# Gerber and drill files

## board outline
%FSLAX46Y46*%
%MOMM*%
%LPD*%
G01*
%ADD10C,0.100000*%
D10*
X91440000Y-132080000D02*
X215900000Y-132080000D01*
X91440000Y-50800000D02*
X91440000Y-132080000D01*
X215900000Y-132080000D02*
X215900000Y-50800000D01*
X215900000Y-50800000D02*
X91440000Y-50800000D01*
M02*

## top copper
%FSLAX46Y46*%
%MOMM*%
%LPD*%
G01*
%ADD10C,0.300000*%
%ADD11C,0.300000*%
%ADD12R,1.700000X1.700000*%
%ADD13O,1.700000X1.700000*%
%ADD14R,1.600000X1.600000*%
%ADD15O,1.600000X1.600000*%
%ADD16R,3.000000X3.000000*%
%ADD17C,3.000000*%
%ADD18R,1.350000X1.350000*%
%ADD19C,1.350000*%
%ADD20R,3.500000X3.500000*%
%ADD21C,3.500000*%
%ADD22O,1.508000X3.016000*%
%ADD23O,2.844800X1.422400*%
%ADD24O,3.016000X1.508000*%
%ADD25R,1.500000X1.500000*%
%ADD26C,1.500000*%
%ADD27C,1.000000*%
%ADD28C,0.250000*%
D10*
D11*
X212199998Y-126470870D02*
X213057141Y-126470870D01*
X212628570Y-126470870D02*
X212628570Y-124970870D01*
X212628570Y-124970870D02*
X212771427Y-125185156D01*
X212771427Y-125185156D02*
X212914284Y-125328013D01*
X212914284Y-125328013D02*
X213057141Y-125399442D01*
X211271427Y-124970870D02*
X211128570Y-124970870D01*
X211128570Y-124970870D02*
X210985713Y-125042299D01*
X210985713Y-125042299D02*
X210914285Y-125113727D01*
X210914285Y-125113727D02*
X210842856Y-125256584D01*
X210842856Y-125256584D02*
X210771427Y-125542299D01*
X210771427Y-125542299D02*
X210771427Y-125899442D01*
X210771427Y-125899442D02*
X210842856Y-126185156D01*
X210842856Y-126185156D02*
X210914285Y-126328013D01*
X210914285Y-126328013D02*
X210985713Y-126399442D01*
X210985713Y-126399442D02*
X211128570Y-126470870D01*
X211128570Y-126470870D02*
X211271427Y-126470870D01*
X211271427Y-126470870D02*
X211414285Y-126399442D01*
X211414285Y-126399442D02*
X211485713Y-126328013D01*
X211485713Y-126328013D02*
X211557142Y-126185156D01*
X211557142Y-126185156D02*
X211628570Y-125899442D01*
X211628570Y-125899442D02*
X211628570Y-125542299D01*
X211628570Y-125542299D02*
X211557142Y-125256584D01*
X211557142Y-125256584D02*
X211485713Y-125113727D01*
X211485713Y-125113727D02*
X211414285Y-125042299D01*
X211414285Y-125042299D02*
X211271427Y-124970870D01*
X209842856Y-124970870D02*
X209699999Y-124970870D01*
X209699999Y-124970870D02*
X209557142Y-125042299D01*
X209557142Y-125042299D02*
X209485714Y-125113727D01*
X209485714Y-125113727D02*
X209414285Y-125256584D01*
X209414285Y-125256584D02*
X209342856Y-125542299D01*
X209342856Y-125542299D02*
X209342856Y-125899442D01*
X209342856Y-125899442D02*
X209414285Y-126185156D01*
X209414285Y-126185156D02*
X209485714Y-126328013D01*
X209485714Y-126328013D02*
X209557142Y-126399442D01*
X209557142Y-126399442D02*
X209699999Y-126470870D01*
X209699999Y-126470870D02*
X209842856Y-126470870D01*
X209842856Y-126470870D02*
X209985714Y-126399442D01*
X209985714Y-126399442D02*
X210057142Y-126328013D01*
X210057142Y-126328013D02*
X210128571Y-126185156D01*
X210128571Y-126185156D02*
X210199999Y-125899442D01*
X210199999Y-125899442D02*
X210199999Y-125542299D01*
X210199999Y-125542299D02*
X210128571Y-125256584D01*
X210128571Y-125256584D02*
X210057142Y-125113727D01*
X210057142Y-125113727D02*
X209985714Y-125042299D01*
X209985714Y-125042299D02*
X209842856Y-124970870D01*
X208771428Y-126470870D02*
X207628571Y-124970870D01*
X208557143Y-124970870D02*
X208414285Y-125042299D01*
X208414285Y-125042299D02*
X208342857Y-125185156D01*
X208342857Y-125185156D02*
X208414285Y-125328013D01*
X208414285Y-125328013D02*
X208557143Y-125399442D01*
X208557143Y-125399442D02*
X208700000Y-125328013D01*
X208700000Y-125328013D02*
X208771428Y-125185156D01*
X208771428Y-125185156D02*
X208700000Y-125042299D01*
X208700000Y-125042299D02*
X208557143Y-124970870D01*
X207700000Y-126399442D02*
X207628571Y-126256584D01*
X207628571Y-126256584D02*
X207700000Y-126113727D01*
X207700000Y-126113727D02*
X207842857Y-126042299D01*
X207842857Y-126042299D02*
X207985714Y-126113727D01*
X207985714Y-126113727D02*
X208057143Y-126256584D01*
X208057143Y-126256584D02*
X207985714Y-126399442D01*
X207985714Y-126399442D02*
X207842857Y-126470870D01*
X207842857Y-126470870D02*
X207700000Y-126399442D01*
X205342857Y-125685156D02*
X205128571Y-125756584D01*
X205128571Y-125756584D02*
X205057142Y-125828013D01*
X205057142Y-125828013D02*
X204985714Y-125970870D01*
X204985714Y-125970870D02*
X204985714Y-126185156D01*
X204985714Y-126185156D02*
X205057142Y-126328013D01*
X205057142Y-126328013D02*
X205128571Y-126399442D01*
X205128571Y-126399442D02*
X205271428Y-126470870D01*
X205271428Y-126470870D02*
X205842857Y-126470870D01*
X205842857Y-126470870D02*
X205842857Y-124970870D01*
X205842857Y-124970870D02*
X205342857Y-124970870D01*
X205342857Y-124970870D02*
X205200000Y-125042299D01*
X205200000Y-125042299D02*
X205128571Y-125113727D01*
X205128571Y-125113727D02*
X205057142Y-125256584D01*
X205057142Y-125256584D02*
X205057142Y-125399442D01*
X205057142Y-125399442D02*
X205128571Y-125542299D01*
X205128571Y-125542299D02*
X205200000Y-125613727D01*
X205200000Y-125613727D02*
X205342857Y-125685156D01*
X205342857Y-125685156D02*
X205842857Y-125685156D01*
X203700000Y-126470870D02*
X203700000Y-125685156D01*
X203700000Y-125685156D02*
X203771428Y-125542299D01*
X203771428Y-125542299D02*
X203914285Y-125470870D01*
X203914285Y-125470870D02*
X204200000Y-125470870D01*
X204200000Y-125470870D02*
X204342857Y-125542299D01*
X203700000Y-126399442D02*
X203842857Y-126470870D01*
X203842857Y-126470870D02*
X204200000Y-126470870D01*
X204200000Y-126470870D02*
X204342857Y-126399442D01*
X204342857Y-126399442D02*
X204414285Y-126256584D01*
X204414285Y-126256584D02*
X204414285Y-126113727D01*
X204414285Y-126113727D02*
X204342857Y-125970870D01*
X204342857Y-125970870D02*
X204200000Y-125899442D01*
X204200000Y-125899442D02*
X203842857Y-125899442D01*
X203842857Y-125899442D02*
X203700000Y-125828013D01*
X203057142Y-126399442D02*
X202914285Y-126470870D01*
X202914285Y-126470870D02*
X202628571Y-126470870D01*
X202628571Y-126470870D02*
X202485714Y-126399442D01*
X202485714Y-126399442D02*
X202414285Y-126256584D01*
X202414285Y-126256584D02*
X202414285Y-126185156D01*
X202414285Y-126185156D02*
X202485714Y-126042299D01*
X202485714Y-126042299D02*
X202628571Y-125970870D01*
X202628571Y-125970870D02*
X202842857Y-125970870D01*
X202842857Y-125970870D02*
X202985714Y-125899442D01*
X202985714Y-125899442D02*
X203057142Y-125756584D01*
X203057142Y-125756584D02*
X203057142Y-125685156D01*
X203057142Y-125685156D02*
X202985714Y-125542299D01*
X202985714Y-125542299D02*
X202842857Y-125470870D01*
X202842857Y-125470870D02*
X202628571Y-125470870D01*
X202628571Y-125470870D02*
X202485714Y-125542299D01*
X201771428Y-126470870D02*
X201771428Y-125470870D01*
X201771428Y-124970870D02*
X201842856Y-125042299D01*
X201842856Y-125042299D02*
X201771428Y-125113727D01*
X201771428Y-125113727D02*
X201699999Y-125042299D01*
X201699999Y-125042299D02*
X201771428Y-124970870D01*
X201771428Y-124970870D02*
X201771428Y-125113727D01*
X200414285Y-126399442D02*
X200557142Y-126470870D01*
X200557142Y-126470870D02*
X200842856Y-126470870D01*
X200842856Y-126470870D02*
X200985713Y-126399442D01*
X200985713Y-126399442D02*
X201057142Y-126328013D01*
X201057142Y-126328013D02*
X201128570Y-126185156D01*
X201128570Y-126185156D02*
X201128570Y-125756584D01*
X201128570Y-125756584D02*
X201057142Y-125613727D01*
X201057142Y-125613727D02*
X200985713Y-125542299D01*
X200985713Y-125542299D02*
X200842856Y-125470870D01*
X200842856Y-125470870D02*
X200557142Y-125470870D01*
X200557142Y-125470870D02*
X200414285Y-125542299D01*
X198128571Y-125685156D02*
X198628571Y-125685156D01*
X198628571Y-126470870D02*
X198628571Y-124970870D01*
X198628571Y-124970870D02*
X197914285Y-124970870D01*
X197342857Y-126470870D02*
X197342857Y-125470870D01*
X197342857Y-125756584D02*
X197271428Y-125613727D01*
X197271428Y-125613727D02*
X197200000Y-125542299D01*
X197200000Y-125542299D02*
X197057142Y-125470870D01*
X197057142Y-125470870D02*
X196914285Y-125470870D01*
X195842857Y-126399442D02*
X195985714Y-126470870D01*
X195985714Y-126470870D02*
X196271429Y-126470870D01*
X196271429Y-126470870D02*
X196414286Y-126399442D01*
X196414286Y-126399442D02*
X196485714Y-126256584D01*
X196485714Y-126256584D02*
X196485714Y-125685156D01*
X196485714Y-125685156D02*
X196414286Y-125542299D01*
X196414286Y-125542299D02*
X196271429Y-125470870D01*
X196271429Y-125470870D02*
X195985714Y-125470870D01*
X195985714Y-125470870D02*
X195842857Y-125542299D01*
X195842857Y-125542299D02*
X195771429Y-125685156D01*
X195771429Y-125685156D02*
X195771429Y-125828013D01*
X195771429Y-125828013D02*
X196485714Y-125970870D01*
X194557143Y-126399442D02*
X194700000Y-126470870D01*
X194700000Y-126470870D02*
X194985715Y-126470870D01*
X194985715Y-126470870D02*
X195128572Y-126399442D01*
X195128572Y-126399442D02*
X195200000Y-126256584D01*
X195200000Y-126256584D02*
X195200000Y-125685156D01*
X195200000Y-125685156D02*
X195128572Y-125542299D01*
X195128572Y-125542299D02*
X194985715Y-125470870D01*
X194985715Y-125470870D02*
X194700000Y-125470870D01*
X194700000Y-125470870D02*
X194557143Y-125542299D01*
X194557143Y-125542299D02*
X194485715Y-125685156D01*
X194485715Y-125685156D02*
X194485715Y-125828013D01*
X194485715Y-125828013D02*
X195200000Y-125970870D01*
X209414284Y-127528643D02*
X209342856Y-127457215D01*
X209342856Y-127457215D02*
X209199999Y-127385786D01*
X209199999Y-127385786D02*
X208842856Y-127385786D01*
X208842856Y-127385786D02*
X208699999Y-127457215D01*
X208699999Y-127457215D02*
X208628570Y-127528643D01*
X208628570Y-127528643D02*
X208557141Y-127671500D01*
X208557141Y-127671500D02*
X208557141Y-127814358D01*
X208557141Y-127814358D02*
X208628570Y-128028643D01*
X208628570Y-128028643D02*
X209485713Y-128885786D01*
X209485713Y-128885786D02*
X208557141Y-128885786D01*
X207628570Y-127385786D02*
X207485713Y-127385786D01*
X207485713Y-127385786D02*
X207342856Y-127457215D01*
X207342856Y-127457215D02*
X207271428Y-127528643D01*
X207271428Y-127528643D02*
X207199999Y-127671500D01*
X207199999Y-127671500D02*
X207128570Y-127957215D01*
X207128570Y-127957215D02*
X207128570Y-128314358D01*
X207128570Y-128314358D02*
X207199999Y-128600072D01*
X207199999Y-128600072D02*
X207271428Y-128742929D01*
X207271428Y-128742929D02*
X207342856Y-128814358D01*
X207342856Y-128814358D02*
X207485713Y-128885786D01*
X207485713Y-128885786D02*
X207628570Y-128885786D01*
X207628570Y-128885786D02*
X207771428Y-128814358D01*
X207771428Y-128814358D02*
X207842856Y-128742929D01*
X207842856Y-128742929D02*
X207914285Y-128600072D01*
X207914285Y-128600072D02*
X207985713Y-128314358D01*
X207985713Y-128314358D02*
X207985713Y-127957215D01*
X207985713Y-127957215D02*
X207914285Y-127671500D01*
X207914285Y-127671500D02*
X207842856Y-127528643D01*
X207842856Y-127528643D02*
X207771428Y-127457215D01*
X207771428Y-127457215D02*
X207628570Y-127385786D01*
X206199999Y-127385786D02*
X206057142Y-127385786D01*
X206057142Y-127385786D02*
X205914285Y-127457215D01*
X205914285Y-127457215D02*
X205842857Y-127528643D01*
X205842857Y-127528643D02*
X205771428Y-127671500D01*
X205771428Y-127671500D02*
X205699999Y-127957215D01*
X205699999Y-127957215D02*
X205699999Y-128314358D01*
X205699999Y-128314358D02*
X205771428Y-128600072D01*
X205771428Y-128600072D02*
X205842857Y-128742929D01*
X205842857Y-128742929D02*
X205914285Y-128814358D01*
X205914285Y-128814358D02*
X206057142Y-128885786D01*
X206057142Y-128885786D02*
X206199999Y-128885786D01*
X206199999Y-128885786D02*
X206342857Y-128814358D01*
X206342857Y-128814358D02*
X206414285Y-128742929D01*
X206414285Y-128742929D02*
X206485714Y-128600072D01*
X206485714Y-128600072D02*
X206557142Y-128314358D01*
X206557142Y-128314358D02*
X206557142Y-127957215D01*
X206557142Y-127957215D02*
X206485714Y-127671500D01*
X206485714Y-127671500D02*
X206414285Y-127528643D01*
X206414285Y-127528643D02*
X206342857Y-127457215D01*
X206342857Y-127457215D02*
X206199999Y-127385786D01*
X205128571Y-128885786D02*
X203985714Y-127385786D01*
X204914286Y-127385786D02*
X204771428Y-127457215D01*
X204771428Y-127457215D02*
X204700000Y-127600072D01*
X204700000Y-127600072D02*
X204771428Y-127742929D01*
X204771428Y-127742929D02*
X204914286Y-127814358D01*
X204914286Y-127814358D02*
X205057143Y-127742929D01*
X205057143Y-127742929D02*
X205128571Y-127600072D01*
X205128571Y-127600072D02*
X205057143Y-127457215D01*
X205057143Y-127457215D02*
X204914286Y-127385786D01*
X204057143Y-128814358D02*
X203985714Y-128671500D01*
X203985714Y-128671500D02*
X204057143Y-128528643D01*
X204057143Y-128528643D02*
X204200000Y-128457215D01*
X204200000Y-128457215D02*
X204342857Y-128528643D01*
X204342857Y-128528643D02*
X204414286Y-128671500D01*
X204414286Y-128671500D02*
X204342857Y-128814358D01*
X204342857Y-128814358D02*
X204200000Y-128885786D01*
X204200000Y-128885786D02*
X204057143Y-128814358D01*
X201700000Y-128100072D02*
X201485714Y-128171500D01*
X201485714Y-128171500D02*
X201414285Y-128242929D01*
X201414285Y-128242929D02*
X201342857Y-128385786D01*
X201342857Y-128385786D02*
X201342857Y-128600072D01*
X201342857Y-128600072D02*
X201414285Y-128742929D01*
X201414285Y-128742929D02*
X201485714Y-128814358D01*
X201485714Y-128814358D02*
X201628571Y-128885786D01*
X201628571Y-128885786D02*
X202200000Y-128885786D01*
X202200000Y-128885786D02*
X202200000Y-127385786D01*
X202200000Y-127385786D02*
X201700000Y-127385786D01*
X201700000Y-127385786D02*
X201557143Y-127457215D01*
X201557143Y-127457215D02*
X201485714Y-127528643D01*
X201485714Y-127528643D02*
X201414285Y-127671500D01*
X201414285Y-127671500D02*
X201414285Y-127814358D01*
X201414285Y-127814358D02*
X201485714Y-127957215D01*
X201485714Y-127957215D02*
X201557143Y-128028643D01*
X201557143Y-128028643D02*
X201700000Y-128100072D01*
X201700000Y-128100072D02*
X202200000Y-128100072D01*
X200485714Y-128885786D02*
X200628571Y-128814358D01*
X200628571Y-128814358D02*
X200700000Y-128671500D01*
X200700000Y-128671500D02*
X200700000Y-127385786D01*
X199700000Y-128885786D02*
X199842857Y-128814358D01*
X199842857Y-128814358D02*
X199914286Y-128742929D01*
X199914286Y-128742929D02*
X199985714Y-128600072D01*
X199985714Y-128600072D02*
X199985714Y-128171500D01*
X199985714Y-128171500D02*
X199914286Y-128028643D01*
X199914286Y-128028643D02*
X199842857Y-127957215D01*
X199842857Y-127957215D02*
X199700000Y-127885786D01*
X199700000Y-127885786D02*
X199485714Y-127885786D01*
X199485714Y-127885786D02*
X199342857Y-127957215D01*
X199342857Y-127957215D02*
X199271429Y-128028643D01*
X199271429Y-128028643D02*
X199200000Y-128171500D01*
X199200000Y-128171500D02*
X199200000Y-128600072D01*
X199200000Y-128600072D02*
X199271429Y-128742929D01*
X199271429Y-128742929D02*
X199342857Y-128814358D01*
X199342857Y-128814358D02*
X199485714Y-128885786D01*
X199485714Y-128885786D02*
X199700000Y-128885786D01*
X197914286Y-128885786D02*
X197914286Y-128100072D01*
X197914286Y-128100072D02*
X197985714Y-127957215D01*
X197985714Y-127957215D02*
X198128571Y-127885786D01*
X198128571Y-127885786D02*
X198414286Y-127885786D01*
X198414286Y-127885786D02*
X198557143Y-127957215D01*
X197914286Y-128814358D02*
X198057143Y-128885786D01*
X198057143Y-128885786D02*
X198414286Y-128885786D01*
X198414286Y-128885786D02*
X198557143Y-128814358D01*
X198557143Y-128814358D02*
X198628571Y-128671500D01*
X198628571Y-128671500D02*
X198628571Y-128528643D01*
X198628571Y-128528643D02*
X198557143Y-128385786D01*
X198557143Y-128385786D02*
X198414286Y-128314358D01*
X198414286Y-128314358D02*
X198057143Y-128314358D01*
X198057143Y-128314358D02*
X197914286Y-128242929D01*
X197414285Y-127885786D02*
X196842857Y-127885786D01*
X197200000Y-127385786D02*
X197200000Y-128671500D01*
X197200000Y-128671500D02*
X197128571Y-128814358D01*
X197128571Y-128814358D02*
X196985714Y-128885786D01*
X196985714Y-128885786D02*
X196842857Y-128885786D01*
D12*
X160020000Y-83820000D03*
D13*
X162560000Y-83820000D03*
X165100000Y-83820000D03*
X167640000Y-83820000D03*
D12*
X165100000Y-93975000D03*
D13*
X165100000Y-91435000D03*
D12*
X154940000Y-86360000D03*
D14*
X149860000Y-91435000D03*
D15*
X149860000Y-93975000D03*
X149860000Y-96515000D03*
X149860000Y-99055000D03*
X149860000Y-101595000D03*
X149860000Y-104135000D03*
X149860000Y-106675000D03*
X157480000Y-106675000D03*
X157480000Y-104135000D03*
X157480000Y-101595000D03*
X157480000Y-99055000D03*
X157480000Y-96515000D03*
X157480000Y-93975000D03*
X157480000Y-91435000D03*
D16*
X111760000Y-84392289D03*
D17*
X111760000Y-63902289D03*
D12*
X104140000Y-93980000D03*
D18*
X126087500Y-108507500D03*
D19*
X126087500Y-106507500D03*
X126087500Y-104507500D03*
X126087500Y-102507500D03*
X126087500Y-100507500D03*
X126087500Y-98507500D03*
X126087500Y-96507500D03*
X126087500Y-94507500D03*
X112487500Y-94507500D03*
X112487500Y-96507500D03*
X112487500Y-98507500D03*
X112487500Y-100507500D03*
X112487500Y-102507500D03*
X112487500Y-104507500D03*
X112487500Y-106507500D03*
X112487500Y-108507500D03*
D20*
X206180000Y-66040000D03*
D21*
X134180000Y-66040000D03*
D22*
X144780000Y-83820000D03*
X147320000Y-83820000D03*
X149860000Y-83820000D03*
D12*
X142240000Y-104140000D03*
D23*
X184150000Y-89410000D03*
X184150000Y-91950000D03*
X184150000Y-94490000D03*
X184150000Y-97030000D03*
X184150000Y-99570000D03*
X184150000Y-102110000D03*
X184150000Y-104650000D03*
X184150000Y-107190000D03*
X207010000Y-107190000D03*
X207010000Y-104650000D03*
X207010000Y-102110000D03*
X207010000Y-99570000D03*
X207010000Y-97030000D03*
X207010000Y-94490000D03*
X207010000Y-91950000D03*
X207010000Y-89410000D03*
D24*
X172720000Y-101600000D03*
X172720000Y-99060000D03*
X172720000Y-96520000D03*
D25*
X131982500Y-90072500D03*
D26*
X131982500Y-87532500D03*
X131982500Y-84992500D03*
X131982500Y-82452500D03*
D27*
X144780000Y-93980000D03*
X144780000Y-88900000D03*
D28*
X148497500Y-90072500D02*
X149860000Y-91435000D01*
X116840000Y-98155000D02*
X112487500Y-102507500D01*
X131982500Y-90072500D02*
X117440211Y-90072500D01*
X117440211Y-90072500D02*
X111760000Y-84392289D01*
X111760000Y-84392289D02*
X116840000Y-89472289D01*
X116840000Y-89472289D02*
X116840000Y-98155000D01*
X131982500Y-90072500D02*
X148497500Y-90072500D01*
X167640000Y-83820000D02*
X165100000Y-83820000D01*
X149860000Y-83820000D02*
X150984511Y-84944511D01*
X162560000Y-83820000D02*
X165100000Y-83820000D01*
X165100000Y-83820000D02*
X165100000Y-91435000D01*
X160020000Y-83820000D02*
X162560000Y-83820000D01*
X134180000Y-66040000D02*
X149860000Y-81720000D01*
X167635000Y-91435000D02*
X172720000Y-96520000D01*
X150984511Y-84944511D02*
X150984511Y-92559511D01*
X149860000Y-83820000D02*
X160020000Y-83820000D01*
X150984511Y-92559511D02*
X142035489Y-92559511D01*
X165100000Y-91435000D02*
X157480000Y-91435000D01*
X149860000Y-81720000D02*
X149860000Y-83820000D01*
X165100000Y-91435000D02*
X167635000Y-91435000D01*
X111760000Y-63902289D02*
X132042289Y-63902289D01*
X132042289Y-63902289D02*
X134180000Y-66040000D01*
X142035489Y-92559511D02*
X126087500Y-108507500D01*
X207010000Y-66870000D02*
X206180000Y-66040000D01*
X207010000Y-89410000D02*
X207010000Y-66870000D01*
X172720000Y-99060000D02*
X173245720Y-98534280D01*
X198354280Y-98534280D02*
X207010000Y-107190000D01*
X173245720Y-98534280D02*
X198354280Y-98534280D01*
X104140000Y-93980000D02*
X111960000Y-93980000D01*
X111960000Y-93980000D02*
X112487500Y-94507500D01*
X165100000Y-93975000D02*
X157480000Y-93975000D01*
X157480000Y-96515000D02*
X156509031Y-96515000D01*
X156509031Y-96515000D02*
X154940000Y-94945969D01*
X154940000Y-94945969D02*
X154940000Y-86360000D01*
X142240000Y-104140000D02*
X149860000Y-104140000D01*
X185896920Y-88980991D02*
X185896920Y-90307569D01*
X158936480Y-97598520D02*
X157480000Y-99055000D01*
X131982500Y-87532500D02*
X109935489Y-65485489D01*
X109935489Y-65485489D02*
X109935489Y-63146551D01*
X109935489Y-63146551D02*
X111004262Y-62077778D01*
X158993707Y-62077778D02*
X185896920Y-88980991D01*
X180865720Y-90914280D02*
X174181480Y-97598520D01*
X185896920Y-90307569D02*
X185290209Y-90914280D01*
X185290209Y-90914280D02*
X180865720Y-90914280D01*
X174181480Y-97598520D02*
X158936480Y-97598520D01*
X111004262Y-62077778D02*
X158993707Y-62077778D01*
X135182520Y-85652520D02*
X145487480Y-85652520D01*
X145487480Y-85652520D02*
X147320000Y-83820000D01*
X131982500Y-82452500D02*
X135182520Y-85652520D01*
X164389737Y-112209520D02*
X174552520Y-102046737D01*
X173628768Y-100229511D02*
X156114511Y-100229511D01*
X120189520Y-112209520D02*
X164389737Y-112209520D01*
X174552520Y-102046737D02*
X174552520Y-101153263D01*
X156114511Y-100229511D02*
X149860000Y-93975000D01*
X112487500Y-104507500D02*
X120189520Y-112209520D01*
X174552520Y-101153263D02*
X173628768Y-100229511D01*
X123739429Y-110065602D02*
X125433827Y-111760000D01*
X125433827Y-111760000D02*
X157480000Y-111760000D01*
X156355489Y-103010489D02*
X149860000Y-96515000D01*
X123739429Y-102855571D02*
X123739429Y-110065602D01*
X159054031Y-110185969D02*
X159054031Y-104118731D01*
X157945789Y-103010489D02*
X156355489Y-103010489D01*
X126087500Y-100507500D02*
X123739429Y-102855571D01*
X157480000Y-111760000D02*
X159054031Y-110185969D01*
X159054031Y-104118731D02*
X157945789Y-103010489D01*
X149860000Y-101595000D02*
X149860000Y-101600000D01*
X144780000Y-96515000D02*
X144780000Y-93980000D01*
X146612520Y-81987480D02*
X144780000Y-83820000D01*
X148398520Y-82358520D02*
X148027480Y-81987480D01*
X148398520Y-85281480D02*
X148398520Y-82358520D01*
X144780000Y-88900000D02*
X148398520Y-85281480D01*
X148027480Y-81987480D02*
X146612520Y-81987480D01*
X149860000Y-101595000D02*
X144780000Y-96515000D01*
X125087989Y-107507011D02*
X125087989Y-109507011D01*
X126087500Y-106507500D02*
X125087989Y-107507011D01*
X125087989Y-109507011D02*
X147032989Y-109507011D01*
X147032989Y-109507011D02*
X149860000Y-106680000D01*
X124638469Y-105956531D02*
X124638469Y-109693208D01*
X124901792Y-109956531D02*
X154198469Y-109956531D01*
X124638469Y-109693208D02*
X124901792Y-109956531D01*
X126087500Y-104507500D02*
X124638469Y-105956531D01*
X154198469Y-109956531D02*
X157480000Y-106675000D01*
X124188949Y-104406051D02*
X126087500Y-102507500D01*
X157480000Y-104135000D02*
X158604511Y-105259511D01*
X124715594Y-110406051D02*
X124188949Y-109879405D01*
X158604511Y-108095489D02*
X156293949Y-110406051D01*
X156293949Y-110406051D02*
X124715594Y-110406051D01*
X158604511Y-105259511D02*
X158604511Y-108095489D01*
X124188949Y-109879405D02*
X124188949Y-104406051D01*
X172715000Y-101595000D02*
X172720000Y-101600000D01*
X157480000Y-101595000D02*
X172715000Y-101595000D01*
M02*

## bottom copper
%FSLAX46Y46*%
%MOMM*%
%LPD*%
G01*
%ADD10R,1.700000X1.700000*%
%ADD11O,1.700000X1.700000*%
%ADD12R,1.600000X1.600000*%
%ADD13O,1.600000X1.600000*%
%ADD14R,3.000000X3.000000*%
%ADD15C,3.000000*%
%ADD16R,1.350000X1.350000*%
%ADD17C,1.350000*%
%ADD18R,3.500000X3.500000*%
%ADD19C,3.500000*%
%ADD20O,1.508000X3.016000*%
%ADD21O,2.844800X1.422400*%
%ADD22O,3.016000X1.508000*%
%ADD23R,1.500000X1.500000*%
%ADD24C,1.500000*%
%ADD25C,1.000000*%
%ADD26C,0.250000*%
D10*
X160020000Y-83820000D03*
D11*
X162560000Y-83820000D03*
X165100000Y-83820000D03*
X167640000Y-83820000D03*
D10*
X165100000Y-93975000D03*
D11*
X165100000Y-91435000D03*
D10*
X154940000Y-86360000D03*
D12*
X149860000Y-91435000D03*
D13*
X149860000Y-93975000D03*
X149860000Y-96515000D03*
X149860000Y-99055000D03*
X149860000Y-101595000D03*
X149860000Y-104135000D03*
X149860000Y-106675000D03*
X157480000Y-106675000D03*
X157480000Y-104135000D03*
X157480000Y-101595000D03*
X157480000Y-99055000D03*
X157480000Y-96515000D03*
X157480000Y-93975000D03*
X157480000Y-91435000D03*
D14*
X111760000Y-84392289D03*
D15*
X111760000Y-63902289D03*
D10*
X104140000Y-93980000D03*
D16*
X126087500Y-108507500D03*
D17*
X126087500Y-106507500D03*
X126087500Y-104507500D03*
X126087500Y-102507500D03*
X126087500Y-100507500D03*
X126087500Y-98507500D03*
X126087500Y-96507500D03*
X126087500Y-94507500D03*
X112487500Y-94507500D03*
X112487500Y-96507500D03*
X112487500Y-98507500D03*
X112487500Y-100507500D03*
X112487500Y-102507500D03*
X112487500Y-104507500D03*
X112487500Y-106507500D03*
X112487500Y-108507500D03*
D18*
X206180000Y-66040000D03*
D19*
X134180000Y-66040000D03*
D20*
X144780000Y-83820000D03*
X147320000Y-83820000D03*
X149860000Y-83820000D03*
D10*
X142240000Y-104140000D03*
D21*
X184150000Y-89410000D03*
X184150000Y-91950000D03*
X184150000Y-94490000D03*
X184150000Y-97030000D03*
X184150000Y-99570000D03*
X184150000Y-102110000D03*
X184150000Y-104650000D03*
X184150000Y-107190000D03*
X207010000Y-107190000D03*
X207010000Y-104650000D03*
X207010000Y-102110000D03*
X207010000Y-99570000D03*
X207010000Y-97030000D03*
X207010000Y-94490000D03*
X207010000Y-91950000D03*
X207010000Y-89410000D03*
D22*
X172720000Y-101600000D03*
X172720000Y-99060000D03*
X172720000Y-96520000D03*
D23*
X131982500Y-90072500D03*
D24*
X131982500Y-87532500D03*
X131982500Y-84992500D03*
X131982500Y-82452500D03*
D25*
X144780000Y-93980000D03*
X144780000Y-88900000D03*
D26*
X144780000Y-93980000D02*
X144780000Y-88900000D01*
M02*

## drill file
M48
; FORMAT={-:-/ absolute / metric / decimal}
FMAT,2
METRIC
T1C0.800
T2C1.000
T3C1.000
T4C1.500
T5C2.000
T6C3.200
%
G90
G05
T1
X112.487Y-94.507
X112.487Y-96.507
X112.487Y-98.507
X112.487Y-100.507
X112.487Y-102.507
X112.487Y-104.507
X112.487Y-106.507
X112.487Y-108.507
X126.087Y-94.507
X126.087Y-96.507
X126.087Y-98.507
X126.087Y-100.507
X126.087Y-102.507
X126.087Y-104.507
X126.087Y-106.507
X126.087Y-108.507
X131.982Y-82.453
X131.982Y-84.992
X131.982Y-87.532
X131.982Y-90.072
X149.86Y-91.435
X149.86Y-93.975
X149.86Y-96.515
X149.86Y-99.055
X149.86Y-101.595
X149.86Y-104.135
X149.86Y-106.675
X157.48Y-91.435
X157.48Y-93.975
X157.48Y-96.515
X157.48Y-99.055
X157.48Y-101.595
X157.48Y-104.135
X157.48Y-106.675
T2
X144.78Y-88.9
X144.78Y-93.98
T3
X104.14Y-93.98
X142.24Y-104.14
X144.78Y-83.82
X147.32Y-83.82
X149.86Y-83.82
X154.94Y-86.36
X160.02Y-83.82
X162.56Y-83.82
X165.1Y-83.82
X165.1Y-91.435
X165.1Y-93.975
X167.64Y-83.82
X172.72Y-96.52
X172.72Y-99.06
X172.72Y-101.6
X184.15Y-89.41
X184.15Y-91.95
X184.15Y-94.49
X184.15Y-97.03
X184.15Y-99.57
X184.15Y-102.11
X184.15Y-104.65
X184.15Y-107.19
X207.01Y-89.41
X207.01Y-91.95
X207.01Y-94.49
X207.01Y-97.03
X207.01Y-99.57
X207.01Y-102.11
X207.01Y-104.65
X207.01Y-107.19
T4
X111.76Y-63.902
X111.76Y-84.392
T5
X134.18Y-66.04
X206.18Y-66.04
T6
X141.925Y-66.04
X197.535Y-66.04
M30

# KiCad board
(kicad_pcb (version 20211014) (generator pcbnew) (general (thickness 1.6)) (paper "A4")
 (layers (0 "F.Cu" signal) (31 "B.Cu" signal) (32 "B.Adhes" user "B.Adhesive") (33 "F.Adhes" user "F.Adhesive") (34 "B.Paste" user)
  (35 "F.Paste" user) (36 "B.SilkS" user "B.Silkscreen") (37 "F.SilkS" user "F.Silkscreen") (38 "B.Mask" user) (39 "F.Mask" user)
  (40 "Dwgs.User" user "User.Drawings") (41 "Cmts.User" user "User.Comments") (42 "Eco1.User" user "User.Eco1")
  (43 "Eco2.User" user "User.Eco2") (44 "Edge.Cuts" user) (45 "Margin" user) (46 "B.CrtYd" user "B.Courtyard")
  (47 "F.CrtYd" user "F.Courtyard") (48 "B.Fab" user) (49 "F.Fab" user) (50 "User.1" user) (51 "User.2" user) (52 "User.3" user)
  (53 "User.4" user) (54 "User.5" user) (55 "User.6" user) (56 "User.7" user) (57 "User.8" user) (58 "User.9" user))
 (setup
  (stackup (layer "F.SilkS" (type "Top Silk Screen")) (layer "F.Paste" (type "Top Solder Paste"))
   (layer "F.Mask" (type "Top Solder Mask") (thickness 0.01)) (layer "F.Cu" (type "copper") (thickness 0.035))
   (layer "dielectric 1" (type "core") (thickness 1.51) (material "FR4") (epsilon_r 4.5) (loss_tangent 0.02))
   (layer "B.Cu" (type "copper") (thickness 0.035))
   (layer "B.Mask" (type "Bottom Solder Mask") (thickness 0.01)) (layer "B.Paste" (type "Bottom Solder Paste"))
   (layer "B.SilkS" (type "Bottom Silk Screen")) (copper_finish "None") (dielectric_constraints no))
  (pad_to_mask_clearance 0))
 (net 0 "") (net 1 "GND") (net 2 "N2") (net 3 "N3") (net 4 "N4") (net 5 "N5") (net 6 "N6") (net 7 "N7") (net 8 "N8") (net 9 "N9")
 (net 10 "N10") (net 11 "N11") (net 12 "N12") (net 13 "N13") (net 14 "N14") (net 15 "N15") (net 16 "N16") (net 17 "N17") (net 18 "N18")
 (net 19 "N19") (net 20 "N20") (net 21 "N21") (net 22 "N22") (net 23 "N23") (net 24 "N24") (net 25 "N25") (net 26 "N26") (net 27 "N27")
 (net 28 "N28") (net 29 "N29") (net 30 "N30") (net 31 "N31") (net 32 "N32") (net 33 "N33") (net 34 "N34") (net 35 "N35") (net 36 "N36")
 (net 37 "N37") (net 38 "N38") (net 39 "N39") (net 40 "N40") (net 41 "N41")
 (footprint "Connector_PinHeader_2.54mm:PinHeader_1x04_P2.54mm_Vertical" (layer "F.Cu") (at 160.02 83.82 90)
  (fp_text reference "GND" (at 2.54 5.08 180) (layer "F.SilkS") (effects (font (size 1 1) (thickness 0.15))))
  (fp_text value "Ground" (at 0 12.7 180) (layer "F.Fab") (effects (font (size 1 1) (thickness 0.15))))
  (pad "1" thru_hole rect (at 0 0 90) (size 1.7 1.7) (drill 1) (layers *.Cu *.Mask) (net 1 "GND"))
  (pad "2" thru_hole oval (at 0 2.54 90) (size 1.7 1.7) (drill 1) (layers *.Cu *.Mask) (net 1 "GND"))
  (pad "3" thru_hole oval (at 0 5.08 90) (size 1.7 1.7) (drill 1) (layers *.Cu *.Mask) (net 1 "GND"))
  (pad "4" thru_hole oval (at 0 7.62 90) (size 1.7 1.7) (drill 1) (layers *.Cu *.Mask) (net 1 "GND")))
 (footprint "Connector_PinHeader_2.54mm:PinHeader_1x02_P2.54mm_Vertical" (layer "F.Cu") (at 165.1 93.975 180)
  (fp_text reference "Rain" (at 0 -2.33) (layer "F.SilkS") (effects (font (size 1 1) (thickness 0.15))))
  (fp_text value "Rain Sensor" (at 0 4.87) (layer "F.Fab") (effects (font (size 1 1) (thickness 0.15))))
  (pad "1" thru_hole rect (at 0 0 180) (size 1.7 1.7) (drill 1) (layers *.Cu *.Mask) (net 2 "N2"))
  (pad "2" thru_hole oval (at 0 2.54 180) (size 1.7 1.7) (drill 1) (layers *.Cu *.Mask) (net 1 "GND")))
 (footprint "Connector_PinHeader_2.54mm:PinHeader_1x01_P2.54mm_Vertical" (layer "F.Cu") (at 154.94 86.36)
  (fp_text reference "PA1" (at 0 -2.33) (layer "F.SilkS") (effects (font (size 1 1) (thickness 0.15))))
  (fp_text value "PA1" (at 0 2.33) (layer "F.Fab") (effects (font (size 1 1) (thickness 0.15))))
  (pad "1" thru_hole rect (at 0 0) (size 1.7 1.7) (drill 1) (layers *.Cu *.Mask) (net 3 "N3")))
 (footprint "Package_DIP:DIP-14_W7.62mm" (layer "F.Cu") (at 149.86 91.435)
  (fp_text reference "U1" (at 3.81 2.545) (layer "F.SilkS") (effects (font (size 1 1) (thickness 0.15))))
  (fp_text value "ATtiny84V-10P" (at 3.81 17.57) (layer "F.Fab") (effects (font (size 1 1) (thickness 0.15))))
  (pad "1" thru_hole rect (at 0 0) (size 1.6 1.6) (drill 0.8) (layers *.Cu *.Mask) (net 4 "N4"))
  (pad "2" thru_hole oval (at 0 2.54) (size 1.6 1.6) (drill 0.8) (layers *.Cu *.Mask) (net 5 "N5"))
  (pad "3" thru_hole oval (at 0 5.08) (size 1.6 1.6) (drill 0.8) (layers *.Cu *.Mask) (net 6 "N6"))
  (pad "4" thru_hole oval (at 0 7.62) (size 1.6 1.6) (drill 0.8) (layers *.Cu *.Mask) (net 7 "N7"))
  (pad "5" thru_hole oval (at 0 10.16) (size 1.6 1.6) (drill 0.8) (layers *.Cu *.Mask) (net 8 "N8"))
  (pad "6" thru_hole oval (at 0 12.7) (size 1.6 1.6) (drill 0.8) (layers *.Cu *.Mask) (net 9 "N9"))
  (pad "7" thru_hole oval (at 0 15.24) (size 1.6 1.6) (drill 0.8) (layers *.Cu *.Mask) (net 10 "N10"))
  (pad "8" thru_hole oval (at 7.62 15.24) (size 1.6 1.6) (drill 0.8) (layers *.Cu *.Mask) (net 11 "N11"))
  (pad "9" thru_hole oval (at 7.62 12.7) (size 1.6 1.6) (drill 0.8) (layers *.Cu *.Mask) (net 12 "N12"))
  (pad "10" thru_hole oval (at 7.62 10.16) (size 1.6 1.6) (drill 0.8) (layers *.Cu *.Mask) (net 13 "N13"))
  (pad "11" thru_hole oval (at 7.62 7.62) (size 1.6 1.6) (drill 0.8) (layers *.Cu *.Mask) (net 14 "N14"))
  (pad "12" thru_hole oval (at 7.62 5.08) (size 1.6 1.6) (drill 0.8) (layers *.Cu *.Mask) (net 3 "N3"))
  (pad "13" thru_hole oval (at 7.62 2.54) (size 1.6 1.6) (drill 0.8) (layers *.Cu *.Mask) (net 2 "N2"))
  (pad "14" thru_hole oval (at 7.62 0) (size 1.6 1.6) (drill 0.8) (layers *.Cu *.Mask) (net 1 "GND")))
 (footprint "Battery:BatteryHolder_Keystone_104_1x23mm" (layer "F.Cu") (at 111.76 84.392289 90)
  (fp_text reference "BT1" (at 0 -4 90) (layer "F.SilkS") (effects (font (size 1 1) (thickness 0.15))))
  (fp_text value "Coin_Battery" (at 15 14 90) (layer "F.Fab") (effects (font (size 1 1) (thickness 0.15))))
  (pad "1" thru_hole rect (at 0 0 90) (size 3 3) (drill 1.5) (layers *.Cu *.Mask) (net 4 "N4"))
  (pad "2" thru_hole circle (at 20.49 0 90) (size 3 3) (drill 1.5) (layers *.Cu *.Mask) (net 1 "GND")))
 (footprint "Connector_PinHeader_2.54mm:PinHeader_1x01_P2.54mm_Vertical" (layer "F.Cu") (at 104.14 93.98)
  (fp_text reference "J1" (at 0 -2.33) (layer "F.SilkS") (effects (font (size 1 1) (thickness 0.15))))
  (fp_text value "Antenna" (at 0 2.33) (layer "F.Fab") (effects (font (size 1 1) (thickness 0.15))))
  (pad "1" thru_hole rect (at 0 0) (size 1.7 1.7) (drill 1) (layers *.Cu *.Mask) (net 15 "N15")))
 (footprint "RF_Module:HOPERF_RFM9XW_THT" (layer "F.Cu") (at 126.0875 108.5075 180)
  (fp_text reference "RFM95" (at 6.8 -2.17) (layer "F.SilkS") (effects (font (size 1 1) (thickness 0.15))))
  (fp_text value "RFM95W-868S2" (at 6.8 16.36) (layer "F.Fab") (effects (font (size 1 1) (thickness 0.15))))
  (pad "1" thru_hole rect (at 0 0 180) (size 1.35 1.35) (drill 0.8) (layers *.Cu *.Mask) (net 1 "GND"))
  (pad "2" thru_hole circle (at 0 2 180) (size 1.35 1.35) (drill 0.8) (layers *.Cu *.Mask) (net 10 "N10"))
  (pad "3" thru_hole circle (at 0 4 180) (size 1.35 1.35) (drill 0.8) (layers *.Cu *.Mask) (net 11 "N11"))
  (pad "4" thru_hole circle (at 0 6 180) (size 1.35 1.35) (drill 0.8) (layers *.Cu *.Mask) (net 12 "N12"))
  (pad "5" thru_hole circle (at 0 8 180) (size 1.35 1.35) (drill 0.8) (layers *.Cu *.Mask) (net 6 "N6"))
  (pad "6" thru_hole circle (at 0 10 180) (size 1.35 1.35) (drill 0.8) (layers *.Cu *.Mask) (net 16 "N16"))
  (pad "7" thru_hole circle (at 0 12 180) (size 1.35 1.35) (drill 0.8) (layers *.Cu *.Mask) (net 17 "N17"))
  (pad "8" thru_hole circle (at 0 14 180) (size 1.35 1.35) (drill 0.8) (layers *.Cu *.Mask) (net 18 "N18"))
  (pad "9" thru_hole circle (at 13.6 14 180) (size 1.35 1.35) (drill 0.8) (layers *.Cu *.Mask) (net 15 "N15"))
  (pad "10" thru_hole circle (at 13.6 12 180) (size 1.35 1.35) (drill 0.8) (layers *.Cu *.Mask) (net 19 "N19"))
  (pad "11" thru_hole circle (at 13.6 10 180) (size 1.35 1.35) (drill 0.8) (layers *.Cu *.Mask) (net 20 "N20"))
  (pad "12" thru_hole circle (at 13.6 8 180) (size 1.35 1.35) (drill 0.8) (layers *.Cu *.Mask) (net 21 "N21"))
  (pad "13" thru_hole circle (at 13.6 6 180) (size 1.35 1.35) (drill 0.8) (layers *.Cu *.Mask) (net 4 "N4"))
  (pad "14" thru_hole circle (at 13.6 4 180) (size 1.35 1.35) (drill 0.8) (layers *.Cu *.Mask) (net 5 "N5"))
  (pad "15" thru_hole circle (at 13.6 2 180) (size 1.35 1.35) (drill 0.8) (layers *.Cu *.Mask) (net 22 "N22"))
  (pad "16" thru_hole circle (at 13.6 0 180) (size 1.35 1.35) (drill 0.8) (layers *.Cu *.Mask) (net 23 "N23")))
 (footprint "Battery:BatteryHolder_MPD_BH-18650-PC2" (layer "F.Cu") (at 206.18 66.04 180)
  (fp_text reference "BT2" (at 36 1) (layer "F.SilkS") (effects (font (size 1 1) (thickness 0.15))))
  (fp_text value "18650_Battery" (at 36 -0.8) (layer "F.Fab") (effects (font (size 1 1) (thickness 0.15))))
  (pad "" np_thru_hole circle (at 8.645 0 180) (size 3.2 3.2) (drill 3.2) (layers *.Cu *.Mask))
  (pad "" np_thru_hole circle (at 64.255 0 180) (size 3.2 3.2) (drill 3.2) (layers *.Cu *.Mask))
  (pad "1" thru_hole rect (at 0 0 180) (size 3.5 3.5) (drill 2) (layers *.Cu *.Mask) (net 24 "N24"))
  (pad "2" thru_hole circle (at 72 0 180) (size 3.5 3.5) (drill 2) (layers *.Cu *.Mask) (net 1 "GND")))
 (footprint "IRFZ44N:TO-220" (layer "F.Cu") (at 147.32 83.82)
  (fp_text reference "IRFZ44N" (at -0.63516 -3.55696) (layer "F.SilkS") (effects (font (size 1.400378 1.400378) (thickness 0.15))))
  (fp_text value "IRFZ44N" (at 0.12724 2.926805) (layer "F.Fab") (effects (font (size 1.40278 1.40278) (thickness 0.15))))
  (pad "1" thru_hole oval locked (at -2.54 0) (size 1.508 3.016) (drill 1) (layers *.Cu *.Mask) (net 8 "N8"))
  (pad "2" thru_hole oval locked (at 0 0) (size 1.508 3.016) (drill 1) (layers *.Cu *.Mask) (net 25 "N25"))
  (pad "3" thru_hole oval locked (at 2.54 0) (size 1.508 3.016) (drill 1) (layers *.Cu *.Mask) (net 1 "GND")))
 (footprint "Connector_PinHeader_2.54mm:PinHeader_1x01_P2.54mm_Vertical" (layer "F.Cu") (at 142.24 104.14)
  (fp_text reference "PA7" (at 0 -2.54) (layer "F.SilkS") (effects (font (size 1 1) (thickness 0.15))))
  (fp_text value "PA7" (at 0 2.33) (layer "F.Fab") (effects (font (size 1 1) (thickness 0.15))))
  (pad "1" thru_hole rect (at 0 0) (size 1.7 1.7) (drill 1) (layers *.Cu *.Mask) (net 9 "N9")))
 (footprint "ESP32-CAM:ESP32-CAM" (layer "F.Cu") (at 195.58 99.57)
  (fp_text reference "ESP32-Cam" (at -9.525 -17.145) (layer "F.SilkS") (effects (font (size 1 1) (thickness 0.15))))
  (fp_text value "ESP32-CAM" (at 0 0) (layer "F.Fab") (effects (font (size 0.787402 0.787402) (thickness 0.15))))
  (pad "P$1" thru_hole oval locked (at -11.43 -10.16) (size 2.8448 1.4224) (drill 1) (layers *.Cu *.Mask) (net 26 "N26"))
  (pad "P$2" thru_hole oval locked (at -11.43 -7.62) (size 2.8448 1.4224) (drill 1) (layers *.Cu *.Mask) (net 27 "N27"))
  (pad "P$3" thru_hole oval locked (at -11.43 -5.08) (size 2.8448 1.4224) (drill 1) (layers *.Cu *.Mask) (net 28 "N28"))
  (pad "P$4" thru_hole oval locked (at -11.43 -2.54) (size 2.8448 1.4224) (drill 1) (layers *.Cu *.Mask) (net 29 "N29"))
  (pad "P$5" thru_hole oval locked (at -11.43 0) (size 2.8448 1.4224) (drill 1) (layers *.Cu *.Mask) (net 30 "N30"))
  (pad "P$6" thru_hole oval locked (at -11.43 2.54) (size 2.8448 1.4224) (drill 1) (layers *.Cu *.Mask) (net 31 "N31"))
  (pad "P$7" thru_hole oval locked (at -11.43 5.08) (size 2.8448 1.4224) (drill 1) (layers *.Cu *.Mask) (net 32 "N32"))
  (pad "P$8" thru_hole oval locked (at -11.43 7.62) (size 2.8448 1.4224) (drill 1) (layers *.Cu *.Mask) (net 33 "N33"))
  (pad "P$9" thru_hole oval locked (at 11.43 7.62) (size 2.8448 1.4224) (drill 1) (layers *.Cu *.Mask) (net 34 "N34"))
  (pad "P$10" thru_hole oval locked (at 11.43 5.08) (size 2.8448 1.4224) (drill 1) (layers *.Cu *.Mask) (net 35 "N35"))
  (pad "P$11" thru_hole oval locked (at 11.43 2.54) (size 2.8448 1.4224) (drill 1) (layers *.Cu *.Mask) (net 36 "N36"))
  (pad "P$12" thru_hole oval locked (at 11.43 0) (size 2.8448 1.4224) (drill 1) (layers *.Cu *.Mask) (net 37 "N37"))
  (pad "P$13" thru_hole oval locked (at 11.43 -2.54) (size 2.8448 1.4224) (drill 1) (layers *.Cu *.Mask) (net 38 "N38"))
  (pad "P$14" thru_hole oval locked (at 11.43 -5.08) (size 2.8448 1.4224) (drill 1) (layers *.Cu *.Mask) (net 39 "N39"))
  (pad "P$15" thru_hole oval locked (at 11.43 -7.62) (size 2.8448 1.4224) (drill 1) (layers *.Cu *.Mask) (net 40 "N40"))
  (pad "P$16" thru_hole oval locked (at 11.43 -10.16) (size 2.8448 1.4224) (drill 1) (layers *.Cu *.Mask) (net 24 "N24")))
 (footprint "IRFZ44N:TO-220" (layer "F.Cu") (at 172.72 99.06 90)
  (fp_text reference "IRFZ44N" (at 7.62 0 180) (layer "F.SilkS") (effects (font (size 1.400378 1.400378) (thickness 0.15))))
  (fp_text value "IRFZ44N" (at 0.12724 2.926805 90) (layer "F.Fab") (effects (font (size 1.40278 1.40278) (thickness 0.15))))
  (pad "1" thru_hole oval locked (at -2.54 0 90) (size 1.508 3.016) (drill 1) (layers *.Cu *.Mask) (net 13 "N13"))
  (pad "2" thru_hole oval locked (at 0 0 90) (size 1.508 3.016) (drill 1) (layers *.Cu *.Mask) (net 34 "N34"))
  (pad "3" thru_hole oval locked (at 2.54 0 90) (size 1.508 3.016) (drill 1) (layers *.Cu *.Mask) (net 1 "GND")))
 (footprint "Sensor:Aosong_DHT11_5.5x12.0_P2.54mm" (layer "F.Cu") (at 131.9825 90.0725 180)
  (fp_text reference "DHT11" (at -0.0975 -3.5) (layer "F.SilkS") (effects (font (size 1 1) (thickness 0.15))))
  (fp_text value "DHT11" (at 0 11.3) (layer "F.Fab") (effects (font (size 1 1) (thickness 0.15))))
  (pad "1" thru_hole rect (at 0 0 180) (size 1.5 1.5) (drill 0.8) (layers *.Cu *.Mask) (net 4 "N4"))
  (pad "2" thru_hole circle (at 0 2.54 180) (size 1.5 1.5) (drill 0.8) (layers *.Cu *.Mask) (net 14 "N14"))
  (pad "3" thru_hole circle (at 0 5.08 180) (size 1.5 1.5) (drill 0.8) (layers *.Cu *.Mask) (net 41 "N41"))
  (pad "4" thru_hole circle (at 0 7.62 180) (size 1.5 1.5) (drill 0.8) (layers *.Cu *.Mask) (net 25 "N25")))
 (gr_line (start 91.44 132.08) (end 215.9 132.08) (layer "Edge.Cuts") (width 0.1))
 (gr_line (start 91.44 50.8) (end 91.44 132.08) (layer "Edge.Cuts") (width 0.1))
 (gr_line (start 215.9 132.08) (end 215.9 50.8) (layer "Edge.Cuts") (width 0.1))
 (gr_line (start 215.9 50.8) (end 91.44 50.8) (layer "Edge.Cuts") (width 0.1))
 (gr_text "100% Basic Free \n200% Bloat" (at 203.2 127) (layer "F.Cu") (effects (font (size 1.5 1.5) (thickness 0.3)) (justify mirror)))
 (segment (start 148.4975 90.0725) (end 149.86 91.435) (width 0.25) (layer "F.Cu") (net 4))
 (segment (start 116.84 98.155) (end 112.4875 102.5075) (width 0.25) (layer "F.Cu") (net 4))
 (segment (start 131.9825 90.0725) (end 117.440211 90.0725) (width 0.25) (layer "F.Cu") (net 4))
 (segment (start 117.440211 90.0725) (end 111.76 84.392289) (width 0.25) (layer "F.Cu") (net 4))
 (segment (start 111.76 84.392289) (end 116.84 89.472289) (width 0.25) (layer "F.Cu") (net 4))
 (segment (start 116.84 89.472289) (end 116.84 98.155) (width 0.25) (layer "F.Cu") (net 4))
 (segment (start 131.9825 90.0725) (end 148.4975 90.0725) (width 0.25) (layer "F.Cu") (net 4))
 (segment (start 167.64 83.82) (end 165.1 83.82) (width 0.25) (layer "F.Cu") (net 1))
 (segment (start 149.86 83.82) (end 150.984511 84.944511) (width 0.25) (layer "F.Cu") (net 1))
 (segment (start 162.56 83.82) (end 165.1 83.82) (width 0.25) (layer "F.Cu") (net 1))
 (segment (start 165.1 83.82) (end 165.1 91.435) (width 0.25) (layer "F.Cu") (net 1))
 (segment (start 160.02 83.82) (end 162.56 83.82) (width 0.25) (layer "F.Cu") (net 1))
 (segment (start 134.18 66.04) (end 149.86 81.72) (width 0.25) (layer "F.Cu") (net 1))
 (segment (start 167.635 91.435) (end 172.72 96.52) (width 0.25) (layer "F.Cu") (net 1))
 (segment (start 150.984511 84.944511) (end 150.984511 92.559511) (width 0.25) (layer "F.Cu") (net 1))
 (segment (start 149.86 83.82) (end 160.02 83.82) (width 0.25) (layer "F.Cu") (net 1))
 (segment (start 150.984511 92.559511) (end 142.035489 92.559511) (width 0.25) (layer "F.Cu") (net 1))
 (segment (start 165.1 91.435) (end 157.48 91.435) (width 0.25) (layer "F.Cu") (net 1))
 (segment (start 149.86 81.72) (end 149.86 83.82) (width 0.25) (layer "F.Cu") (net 1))
 (segment (start 165.1 91.435) (end 167.635 91.435) (width 0.25) (layer "F.Cu") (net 1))
 (segment (start 111.76 63.902289) (end 132.042289 63.902289) (width 0.25) (layer "F.Cu") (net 1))
 (segment (start 132.042289 63.902289) (end 134.18 66.04) (width 0.25) (layer "F.Cu") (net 1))
 (segment (start 142.035489 92.559511) (end 126.0875 108.5075) (width 0.25) (layer "F.Cu") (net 1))
 (segment (start 207.01 66.87) (end 206.18 66.04) (width 0.25) (layer "F.Cu") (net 24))
 (segment (start 207.01 89.41) (end 207.01 66.87) (width 0.25) (layer "F.Cu") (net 24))
 (segment (start 172.72 99.06) (end 173.24572 98.53428) (width 0.25) (layer "F.Cu") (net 34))
 (segment (start 198.35428 98.53428) (end 207.01 107.19) (width 0.25) (layer "F.Cu") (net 34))
 (segment (start 173.24572 98.53428) (end 198.35428 98.53428) (width 0.25) (layer "F.Cu") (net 34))
 (segment (start 104.14 93.98) (end 111.96 93.98) (width 0.25) (layer "F.Cu") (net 15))
 (segment (start 111.96 93.98) (end 112.4875 94.5075) (width 0.25) (layer "F.Cu") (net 15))
 (segment (start 165.1 93.975) (end 157.48 93.975) (width 0.25) (layer "F.Cu") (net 2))
 (segment (start 157.48 96.515) (end 156.509031 96.515) (width 0.25) (layer "F.Cu") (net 3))
 (segment (start 156.509031 96.515) (end 154.94 94.945969) (width 0.25) (layer "F.Cu") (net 3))
 (segment (start 154.94 94.945969) (end 154.94 86.36) (width 0.25) (layer "F.Cu") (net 3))
 (segment (start 142.24 104.14) (end 149.86 104.14) (width 0.25) (layer "F.Cu") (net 9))
 (segment (start 185.89692 88.980991) (end 185.89692 90.307569) (width 0.25) (layer "F.Cu") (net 14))
 (segment (start 158.93648 97.59852) (end 157.48 99.055) (width 0.25) (layer "F.Cu") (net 14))
 (segment (start 131.9825 87.5325) (end 109.935489 65.485489) (width 0.25) (layer "F.Cu") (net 14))
 (segment (start 109.935489 65.485489) (end 109.935489 63.146551) (width 0.25) (layer "F.Cu") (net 14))
 (segment (start 109.935489 63.146551) (end 111.004262 62.077778) (width 0.25) (layer "F.Cu") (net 14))
 (segment (start 158.993707 62.077778) (end 185.89692 88.980991) (width 0.25) (layer "F.Cu") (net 14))
 (segment (start 180.86572 90.91428) (end 174.18148 97.59852) (width 0.25) (layer "F.Cu") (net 14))
 (segment (start 185.89692 90.307569) (end 185.290209 90.91428) (width 0.25) (layer "F.Cu") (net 14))
 (segment (start 185.290209 90.91428) (end 180.86572 90.91428) (width 0.25) (layer "F.Cu") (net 14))
 (segment (start 174.18148 97.59852) (end 158.93648 97.59852) (width 0.25) (layer "F.Cu") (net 14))
 (segment (start 111.004262 62.077778) (end 158.993707 62.077778) (width 0.25) (layer "F.Cu") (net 14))
 (segment (start 135.18252 85.65252) (end 145.48748 85.65252) (width 0.25) (layer "F.Cu") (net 25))
 (segment (start 145.48748 85.65252) (end 147.32 83.82) (width 0.25) (layer "F.Cu") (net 25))
 (segment (start 131.9825 82.4525) (end 135.18252 85.65252) (width 0.25) (layer "F.Cu") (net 25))
 (segment (start 164.389737 112.20952) (end 174.55252 102.046737) (width 0.25) (layer "F.Cu") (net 5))
 (segment (start 173.628768 100.229511) (end 156.114511 100.229511) (width 0.25) (layer "F.Cu") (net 5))
 (segment (start 120.18952 112.20952) (end 164.389737 112.20952) (width 0.25) (layer "F.Cu") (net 5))
 (segment (start 174.55252 102.046737) (end 174.55252 101.153263) (width 0.25) (layer "F.Cu") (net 5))
 (segment (start 156.114511 100.229511) (end 149.86 93.975) (width 0.25) (layer "F.Cu") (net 5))
 (segment (start 112.4875 104.5075) (end 120.18952 112.20952) (width 0.25) (layer "F.Cu") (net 5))
 (segment (start 174.55252 101.153263) (end 173.628768 100.229511) (width 0.25) (layer "F.Cu") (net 5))
 (segment (start 123.739429 110.065602) (end 125.433827 111.76) (width 0.25) (layer "F.Cu") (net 6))
 (segment (start 125.433827 111.76) (end 157.48 111.76) (width 0.25) (layer "F.Cu") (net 6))
 (segment (start 156.355489 103.010489) (end 149.86 96.515) (width 0.25) (layer "F.Cu") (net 6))
 (segment (start 123.739429 102.855571) (end 123.739429 110.065602) (width 0.25) (layer "F.Cu") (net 6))
 (segment (start 159.054031 110.185969) (end 159.054031 104.118731) (width 0.25) (layer "F.Cu") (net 6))
 (segment (start 157.945789 103.010489) (end 156.355489 103.010489) (width 0.25) (layer "F.Cu") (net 6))
 (segment (start 126.0875 100.5075) (end 123.739429 102.855571) (width 0.25) (layer "F.Cu") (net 6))
 (segment (start 157.48 111.76) (end 159.054031 110.185969) (width 0.25) (layer "F.Cu") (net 6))
 (segment (start 159.054031 104.118731) (end 157.945789 103.010489) (width 0.25) (layer "F.Cu") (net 6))
 (segment (start 149.86 101.595) (end 149.86 101.6) (width 0.25) (layer "F.Cu") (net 8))
 (segment (start 144.78 96.515) (end 144.78 93.98) (width 0.25) (layer "F.Cu") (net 8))
 (segment (start 146.61252 81.98748) (end 144.78 83.82) (width 0.25) (layer "F.Cu") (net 8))
 (segment (start 148.39852 82.35852) (end 148.02748 81.98748) (width 0.25) (layer "F.Cu") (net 8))
 (segment (start 148.39852 85.28148) (end 148.39852 82.35852) (width 0.25) (layer "F.Cu") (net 8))
 (segment (start 144.78 88.9) (end 148.39852 85.28148) (width 0.25) (layer "F.Cu") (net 8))
 (segment (start 148.02748 81.98748) (end 146.61252 81.98748) (width 0.25) (layer "F.Cu") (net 8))
 (segment (start 149.86 101.595) (end 144.78 96.515) (width 0.25) (layer "F.Cu") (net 8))
 (via (at 144.78 93.98) (size 1) (drill 1) (layers "F.Cu" "B.Cu") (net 8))
 (via (at 144.78 88.9) (size 1) (drill 1) (layers "F.Cu" "B.Cu") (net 8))
 (segment (start 144.78 93.98) (end 144.78 88.9) (width 0.25) (layer "B.Cu") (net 8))
 (segment (start 125.087989 107.507011) (end 125.087989 109.507011) (width 0.25) (layer "F.Cu") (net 10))
 (segment (start 126.0875 106.5075) (end 125.087989 107.507011) (width 0.25) (layer "F.Cu") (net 10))
 (segment (start 125.087989 109.507011) (end 147.032989 109.507011) (width 0.25) (layer "F.Cu") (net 10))
 (segment (start 147.032989 109.507011) (end 149.86 106.68) (width 0.25) (layer "F.Cu") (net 10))
 (segment (start 124.638469 105.956531) (end 124.638469 109.693208) (width 0.25) (layer "F.Cu") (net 11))
 (segment (start 124.901792 109.956531) (end 154.198469 109.956531) (width 0.25) (layer "F.Cu") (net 11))
 (segment (start 124.638469 109.693208) (end 124.901792 109.956531) (width 0.25) (layer "F.Cu") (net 11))
 (segment (start 126.0875 104.5075) (end 124.638469 105.956531) (width 0.25) (layer "F.Cu") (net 11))
 (segment (start 154.198469 109.956531) (end 157.48 106.675) (width 0.25) (layer "F.Cu") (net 11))
 (segment (start 124.188949 104.406051) (end 126.0875 102.5075) (width 0.25) (layer "F.Cu") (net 12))
 (segment (start 157.48 104.135) (end 158.604511 105.259511) (width 0.25) (layer "F.Cu") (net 12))
 (segment (start 124.715594 110.406051) (end 124.188949 109.879405) (width 0.25) (layer "F.Cu") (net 12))
 (segment (start 158.604511 108.095489) (end 156.293949 110.406051) (width 0.25) (layer "F.Cu") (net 12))
 (segment (start 156.293949 110.406051) (end 124.715594 110.406051) (width 0.25) (layer "F.Cu") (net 12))
 (segment (start 158.604511 105.259511) (end 158.604511 108.095489) (width 0.25) (layer "F.Cu") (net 12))
 (segment (start 124.188949 109.879405) (end 124.188949 104.406051) (width 0.25) (layer "F.Cu") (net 12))
 (segment (start 172.715 101.595) (end 172.72 101.6) (width 0.25) (layer "F.Cu") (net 13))
 (segment (start 157.48 101.595) (end 172.715 101.595) (width 0.25) (layer "F.Cu") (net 13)))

